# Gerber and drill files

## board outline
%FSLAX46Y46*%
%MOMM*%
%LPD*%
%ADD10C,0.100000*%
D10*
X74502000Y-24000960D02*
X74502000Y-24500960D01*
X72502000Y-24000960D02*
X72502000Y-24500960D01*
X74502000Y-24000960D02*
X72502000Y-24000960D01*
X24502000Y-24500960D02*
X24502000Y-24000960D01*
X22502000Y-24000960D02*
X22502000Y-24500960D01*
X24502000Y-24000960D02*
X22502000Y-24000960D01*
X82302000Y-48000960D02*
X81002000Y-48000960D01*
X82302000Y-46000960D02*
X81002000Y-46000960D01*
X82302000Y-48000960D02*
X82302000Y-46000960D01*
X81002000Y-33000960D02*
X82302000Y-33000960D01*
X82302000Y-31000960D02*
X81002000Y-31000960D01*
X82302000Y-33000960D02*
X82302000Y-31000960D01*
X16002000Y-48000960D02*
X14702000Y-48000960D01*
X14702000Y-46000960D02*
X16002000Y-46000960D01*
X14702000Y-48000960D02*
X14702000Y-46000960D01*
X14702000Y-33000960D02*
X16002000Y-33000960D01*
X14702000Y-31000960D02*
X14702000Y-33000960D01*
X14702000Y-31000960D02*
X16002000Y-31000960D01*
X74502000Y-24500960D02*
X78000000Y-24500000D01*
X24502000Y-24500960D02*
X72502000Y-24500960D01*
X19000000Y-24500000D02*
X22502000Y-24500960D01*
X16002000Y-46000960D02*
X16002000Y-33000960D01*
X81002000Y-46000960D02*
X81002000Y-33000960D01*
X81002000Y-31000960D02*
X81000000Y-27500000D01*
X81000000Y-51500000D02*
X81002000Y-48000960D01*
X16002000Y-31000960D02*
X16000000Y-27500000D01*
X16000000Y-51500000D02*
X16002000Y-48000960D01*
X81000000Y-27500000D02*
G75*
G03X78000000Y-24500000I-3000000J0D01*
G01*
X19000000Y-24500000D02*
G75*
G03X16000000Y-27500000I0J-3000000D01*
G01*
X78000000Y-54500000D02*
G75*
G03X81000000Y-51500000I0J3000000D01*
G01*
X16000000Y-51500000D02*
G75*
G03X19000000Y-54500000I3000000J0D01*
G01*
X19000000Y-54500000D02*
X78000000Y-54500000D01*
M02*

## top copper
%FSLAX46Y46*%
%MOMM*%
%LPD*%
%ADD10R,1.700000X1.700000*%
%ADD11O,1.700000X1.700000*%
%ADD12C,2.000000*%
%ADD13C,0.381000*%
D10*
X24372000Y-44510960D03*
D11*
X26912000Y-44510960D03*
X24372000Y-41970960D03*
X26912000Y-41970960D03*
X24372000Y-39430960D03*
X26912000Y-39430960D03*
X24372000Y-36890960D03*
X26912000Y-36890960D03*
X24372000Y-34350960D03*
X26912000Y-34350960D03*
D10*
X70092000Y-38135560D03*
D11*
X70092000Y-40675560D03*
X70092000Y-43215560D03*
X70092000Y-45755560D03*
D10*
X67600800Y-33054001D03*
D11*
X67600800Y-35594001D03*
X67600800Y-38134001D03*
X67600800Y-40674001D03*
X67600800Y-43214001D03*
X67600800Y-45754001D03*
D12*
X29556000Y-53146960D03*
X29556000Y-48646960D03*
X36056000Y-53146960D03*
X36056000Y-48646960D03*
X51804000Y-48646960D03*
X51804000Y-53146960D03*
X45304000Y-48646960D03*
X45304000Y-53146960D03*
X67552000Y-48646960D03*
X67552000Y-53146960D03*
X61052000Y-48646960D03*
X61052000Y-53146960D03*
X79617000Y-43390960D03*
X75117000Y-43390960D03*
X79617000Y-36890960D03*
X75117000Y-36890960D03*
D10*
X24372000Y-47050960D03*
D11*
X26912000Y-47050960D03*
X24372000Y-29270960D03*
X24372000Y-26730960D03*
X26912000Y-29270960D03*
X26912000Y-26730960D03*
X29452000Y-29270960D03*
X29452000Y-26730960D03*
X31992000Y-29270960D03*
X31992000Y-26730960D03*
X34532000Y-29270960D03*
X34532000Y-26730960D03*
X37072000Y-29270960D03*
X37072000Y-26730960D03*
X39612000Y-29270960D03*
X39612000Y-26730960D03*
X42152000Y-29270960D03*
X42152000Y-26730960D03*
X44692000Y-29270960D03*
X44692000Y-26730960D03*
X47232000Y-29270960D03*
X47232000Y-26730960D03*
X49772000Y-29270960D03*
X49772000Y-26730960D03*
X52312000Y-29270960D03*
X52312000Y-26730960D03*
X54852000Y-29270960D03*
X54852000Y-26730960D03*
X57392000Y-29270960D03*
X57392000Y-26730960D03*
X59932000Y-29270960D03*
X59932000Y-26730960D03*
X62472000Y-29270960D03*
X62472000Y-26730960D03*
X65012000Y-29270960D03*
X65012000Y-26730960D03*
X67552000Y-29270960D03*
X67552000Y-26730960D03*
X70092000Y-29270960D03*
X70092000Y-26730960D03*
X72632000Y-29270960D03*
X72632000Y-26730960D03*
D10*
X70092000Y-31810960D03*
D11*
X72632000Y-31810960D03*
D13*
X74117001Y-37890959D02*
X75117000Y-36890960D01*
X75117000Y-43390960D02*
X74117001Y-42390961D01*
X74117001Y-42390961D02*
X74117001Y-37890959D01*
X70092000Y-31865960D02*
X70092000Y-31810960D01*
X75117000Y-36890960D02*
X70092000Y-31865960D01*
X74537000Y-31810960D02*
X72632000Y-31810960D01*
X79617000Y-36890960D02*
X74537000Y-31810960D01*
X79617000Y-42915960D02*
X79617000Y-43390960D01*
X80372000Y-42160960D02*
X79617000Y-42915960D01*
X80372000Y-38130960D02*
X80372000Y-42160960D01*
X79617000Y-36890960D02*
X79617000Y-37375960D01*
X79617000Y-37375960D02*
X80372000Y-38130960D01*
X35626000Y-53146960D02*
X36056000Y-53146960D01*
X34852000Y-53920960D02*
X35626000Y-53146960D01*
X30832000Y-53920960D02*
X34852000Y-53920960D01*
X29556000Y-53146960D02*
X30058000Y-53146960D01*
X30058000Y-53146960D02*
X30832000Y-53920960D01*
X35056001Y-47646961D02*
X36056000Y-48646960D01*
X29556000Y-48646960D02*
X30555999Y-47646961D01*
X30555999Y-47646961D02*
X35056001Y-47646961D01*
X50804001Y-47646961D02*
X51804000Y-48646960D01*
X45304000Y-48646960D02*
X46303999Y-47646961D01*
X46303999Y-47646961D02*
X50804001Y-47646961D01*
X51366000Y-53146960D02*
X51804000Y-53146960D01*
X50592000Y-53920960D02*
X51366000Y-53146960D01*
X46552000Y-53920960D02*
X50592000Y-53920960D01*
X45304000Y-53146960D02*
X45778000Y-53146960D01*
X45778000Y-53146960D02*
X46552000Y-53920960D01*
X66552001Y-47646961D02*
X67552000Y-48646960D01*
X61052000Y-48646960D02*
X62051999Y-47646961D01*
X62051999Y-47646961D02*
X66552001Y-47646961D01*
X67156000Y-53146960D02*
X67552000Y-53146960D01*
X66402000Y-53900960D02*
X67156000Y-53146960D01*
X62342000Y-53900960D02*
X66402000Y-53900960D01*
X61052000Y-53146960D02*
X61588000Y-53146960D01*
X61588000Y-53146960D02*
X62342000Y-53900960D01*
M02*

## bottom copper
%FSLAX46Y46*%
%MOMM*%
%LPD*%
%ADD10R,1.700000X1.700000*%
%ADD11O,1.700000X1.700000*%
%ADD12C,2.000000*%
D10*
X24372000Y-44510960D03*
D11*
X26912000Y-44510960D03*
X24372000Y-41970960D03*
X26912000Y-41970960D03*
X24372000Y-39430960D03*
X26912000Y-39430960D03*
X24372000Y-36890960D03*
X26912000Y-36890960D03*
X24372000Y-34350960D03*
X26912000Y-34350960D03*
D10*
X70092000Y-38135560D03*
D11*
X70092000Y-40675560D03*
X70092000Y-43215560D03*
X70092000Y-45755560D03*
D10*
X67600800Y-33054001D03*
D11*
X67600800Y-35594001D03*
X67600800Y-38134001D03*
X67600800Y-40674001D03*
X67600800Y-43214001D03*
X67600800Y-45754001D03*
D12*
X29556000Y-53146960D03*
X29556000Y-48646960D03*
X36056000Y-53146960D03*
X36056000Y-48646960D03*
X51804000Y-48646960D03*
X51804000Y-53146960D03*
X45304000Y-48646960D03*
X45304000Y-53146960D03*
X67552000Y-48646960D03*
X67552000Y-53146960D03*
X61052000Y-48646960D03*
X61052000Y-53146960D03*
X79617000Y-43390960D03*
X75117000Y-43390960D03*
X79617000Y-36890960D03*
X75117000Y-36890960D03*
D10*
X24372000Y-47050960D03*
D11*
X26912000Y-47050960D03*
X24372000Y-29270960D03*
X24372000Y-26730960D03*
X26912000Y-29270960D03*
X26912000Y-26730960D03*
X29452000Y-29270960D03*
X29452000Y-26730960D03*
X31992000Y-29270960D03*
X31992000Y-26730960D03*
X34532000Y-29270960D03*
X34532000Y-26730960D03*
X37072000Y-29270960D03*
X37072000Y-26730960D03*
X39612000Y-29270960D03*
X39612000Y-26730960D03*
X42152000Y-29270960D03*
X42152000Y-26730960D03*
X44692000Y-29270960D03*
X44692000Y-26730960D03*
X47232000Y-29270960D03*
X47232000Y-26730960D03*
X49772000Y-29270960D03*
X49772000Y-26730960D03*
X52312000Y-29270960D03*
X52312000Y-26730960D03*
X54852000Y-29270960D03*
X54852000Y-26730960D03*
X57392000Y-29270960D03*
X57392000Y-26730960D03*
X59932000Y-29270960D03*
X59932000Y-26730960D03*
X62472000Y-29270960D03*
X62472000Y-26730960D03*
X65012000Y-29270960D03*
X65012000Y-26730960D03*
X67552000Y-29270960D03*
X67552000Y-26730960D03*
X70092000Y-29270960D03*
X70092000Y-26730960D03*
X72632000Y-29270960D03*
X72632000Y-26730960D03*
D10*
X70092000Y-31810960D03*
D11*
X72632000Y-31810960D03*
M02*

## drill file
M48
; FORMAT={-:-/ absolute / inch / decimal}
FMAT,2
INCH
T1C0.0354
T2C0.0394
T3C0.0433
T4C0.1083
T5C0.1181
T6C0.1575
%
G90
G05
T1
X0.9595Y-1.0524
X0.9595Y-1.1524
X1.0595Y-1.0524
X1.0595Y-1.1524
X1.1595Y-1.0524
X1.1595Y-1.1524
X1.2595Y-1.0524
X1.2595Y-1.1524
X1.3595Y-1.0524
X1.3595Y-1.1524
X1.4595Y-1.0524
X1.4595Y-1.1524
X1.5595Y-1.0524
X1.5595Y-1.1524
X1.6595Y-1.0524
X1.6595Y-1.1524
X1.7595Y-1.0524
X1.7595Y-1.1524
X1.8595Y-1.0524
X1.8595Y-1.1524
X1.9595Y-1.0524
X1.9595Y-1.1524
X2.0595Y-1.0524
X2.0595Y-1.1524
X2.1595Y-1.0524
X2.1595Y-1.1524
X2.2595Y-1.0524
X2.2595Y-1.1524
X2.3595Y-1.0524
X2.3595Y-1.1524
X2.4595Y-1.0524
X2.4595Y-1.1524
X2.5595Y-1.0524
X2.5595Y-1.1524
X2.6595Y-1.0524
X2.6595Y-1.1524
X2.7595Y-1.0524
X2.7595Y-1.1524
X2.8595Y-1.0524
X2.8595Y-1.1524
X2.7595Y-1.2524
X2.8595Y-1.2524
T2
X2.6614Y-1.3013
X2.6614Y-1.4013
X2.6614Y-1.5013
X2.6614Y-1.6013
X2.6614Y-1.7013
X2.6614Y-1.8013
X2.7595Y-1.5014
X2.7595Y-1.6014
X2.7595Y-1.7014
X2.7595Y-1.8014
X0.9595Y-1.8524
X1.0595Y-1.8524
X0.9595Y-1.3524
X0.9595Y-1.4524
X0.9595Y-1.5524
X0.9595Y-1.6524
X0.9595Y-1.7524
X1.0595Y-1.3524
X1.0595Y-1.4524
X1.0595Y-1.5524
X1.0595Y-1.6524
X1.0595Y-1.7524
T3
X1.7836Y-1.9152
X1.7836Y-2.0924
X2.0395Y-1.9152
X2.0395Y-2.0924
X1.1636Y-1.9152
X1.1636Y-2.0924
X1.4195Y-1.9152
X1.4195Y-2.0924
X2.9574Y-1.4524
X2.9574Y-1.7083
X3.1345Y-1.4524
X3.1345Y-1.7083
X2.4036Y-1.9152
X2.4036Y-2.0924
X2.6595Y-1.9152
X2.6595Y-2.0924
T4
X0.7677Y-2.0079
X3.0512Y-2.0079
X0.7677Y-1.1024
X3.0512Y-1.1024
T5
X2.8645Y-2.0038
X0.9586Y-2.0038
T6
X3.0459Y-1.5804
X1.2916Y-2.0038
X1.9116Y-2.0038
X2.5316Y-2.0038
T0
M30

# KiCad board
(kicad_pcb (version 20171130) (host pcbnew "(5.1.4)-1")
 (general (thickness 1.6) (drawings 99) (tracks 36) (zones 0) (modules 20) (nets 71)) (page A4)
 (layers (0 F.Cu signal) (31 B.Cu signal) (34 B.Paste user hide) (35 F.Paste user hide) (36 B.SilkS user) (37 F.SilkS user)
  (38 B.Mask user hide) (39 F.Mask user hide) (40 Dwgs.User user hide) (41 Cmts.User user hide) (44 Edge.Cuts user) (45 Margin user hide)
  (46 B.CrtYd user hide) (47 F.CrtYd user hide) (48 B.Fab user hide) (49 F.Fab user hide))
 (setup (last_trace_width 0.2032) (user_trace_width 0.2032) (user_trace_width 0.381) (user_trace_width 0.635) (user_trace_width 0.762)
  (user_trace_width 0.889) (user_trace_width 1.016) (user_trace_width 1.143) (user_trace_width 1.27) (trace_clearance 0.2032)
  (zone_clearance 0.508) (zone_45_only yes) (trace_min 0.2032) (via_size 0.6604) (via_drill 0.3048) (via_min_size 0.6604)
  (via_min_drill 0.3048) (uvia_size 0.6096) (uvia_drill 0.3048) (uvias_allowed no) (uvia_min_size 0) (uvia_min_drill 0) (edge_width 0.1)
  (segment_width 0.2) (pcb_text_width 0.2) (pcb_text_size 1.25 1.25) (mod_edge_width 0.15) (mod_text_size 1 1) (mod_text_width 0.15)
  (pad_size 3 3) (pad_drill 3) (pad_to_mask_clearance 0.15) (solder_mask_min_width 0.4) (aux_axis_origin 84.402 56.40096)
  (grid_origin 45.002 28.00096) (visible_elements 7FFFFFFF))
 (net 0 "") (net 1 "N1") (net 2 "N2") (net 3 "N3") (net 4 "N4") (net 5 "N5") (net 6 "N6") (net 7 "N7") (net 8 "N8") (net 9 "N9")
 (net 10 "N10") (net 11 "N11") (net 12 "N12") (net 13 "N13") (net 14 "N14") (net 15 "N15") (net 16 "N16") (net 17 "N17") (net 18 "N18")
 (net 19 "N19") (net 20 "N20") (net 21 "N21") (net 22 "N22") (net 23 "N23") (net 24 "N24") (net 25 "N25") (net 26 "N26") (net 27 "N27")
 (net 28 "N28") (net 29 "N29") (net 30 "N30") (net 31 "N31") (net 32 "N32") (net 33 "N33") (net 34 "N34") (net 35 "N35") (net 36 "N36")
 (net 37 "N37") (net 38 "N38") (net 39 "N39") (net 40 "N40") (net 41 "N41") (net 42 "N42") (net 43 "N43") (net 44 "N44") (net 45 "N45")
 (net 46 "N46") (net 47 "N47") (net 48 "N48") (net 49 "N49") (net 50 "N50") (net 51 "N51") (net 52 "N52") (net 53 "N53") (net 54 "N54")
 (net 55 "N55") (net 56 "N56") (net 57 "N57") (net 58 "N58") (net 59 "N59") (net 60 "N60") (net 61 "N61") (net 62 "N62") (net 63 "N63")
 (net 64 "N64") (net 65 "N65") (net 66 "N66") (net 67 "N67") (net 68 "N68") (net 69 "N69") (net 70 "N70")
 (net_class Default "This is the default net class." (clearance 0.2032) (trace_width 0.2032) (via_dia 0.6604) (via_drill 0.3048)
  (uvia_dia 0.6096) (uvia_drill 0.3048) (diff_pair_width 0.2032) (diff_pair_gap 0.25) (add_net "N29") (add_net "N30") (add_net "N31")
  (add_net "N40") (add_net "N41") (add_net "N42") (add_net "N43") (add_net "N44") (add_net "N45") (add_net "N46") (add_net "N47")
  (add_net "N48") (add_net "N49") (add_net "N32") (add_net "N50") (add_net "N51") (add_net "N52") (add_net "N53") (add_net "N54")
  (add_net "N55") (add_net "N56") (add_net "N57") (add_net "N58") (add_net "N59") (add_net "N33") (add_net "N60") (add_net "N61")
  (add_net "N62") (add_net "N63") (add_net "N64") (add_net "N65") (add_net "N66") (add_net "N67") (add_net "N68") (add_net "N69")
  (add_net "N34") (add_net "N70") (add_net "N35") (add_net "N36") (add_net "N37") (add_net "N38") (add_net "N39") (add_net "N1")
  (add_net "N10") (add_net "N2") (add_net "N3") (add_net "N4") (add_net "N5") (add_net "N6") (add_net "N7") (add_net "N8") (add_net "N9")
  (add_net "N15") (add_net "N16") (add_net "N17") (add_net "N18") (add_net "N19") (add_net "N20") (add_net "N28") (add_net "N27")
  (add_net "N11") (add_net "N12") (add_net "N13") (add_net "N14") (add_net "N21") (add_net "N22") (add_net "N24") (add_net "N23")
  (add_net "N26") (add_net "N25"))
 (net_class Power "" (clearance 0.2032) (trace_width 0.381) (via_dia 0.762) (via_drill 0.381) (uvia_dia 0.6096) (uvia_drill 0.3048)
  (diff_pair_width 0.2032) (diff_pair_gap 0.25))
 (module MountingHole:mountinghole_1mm (layer F.Cu) (at 77.33862 39.95166)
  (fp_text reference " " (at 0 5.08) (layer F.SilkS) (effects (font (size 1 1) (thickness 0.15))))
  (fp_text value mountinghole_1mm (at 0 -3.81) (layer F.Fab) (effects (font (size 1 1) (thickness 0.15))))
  (pad "" np_thru_hole circle (at 0.02838 0.1893) (size 4 4) (drill 4) (layers *.Cu *.Mask) (zone_connect 0)))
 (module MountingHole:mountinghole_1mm (layer F.Cu) (at 24.35676 50.90668)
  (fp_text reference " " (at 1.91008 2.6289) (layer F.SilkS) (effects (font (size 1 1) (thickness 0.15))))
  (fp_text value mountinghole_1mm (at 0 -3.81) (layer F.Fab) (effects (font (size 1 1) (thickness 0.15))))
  (pad "" np_thru_hole circle (at -0.00776 -0.00972) (size 3 3) (drill 3) (layers *.Cu *.Mask)))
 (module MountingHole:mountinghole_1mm (layer F.Cu) (at 72.74376 50.90668)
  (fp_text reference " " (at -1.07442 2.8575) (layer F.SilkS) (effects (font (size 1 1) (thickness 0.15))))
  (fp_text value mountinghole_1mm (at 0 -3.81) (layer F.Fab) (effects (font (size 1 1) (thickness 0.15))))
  (pad "" np_thru_hole circle (at 0.01524 -0.00972) (size 3 3) (drill 3) (layers *.Cu *.Mask)))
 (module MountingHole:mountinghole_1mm (layer F.Cu) (at 64.29826 50.90414)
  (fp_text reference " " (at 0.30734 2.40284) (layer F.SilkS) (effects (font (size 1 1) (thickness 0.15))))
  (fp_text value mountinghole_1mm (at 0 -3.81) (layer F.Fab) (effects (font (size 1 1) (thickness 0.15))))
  (pad "" np_thru_hole circle (at 0.00374 -0.00718) (size 4 4) (drill 4) (layers *.Cu *.Mask) (zone_connect 0)))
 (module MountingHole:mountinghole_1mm (layer F.Cu) (at 48.51978 50.90414)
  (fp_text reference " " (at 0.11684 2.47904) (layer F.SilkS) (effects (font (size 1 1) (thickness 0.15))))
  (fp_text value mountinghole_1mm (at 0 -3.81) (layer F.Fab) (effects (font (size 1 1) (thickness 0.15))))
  (pad "" np_thru_hole circle (at 0.03422 -0.00718) (size 4 4) (drill 4) (layers *.Cu *.Mask) (zone_connect 0)))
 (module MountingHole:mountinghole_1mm (layer F.Cu) (at 32.78956 50.89398)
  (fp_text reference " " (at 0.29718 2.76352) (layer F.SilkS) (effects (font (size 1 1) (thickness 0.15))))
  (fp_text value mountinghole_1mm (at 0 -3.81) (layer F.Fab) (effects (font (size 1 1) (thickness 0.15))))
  (pad "" np_thru_hole circle (at 0.01644 0.00298) (size 4 4) (drill 4) (layers *.Cu *.Mask) (zone_connect 0)))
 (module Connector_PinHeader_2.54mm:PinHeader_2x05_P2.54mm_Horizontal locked (layer B.Cu) (at 24.372 44.51096)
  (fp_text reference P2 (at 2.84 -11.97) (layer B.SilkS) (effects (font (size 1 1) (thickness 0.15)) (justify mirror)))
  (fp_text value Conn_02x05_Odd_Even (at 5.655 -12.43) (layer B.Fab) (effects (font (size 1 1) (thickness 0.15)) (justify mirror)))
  (pad 1 thru_hole rect (at 0 0) (size 1.7 1.7) (drill 1) (layers *.Cu *.Mask) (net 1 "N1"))
  (pad 2 thru_hole oval (at 2.54 0) (size 1.7 1.7) (drill 1) (layers *.Cu *.Mask) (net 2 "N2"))
  (pad 3 thru_hole oval (at 0 -2.54) (size 1.7 1.7) (drill 1) (layers *.Cu *.Mask) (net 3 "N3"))
  (pad 4 thru_hole oval (at 2.54 -2.54) (size 1.7 1.7) (drill 1) (layers *.Cu *.Mask) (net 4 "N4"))
  (pad 5 thru_hole oval (at 0 -5.08) (size 1.7 1.7) (drill 1) (layers *.Cu *.Mask) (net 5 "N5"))
  (pad 6 thru_hole oval (at 2.54 -5.08) (size 1.7 1.7) (drill 1) (layers *.Cu *.Mask) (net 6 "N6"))
  (pad 7 thru_hole oval (at 0 -7.62) (size 1.7 1.7) (drill 1) (layers *.Cu *.Mask) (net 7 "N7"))
  (pad 8 thru_hole oval (at 2.54 -7.62) (size 1.7 1.7) (drill 1) (layers *.Cu *.Mask) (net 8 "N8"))
  (pad 9 thru_hole oval (at 0 -10.16) (size 1.7 1.7) (drill 1) (layers *.Cu *.Mask) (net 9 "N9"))
  (pad 10 thru_hole oval (at 2.54 -10.16) (size 1.7 1.7) (drill 1) (layers *.Cu *.Mask) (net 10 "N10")))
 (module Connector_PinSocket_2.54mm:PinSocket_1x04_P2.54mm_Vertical (layer B.Cu) (at 70.092 38.13556 180)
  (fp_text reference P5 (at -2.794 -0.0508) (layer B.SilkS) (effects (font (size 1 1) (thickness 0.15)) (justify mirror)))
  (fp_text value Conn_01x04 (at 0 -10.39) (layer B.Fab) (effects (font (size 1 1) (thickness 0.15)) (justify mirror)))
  (pad 1 thru_hole rect (at 0 0 180) (size 1.7 1.7) (drill 1) (layers *.Cu *.Mask) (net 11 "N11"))
  (pad 2 thru_hole oval (at 0 -2.54 180) (size 1.7 1.7) (drill 1) (layers *.Cu *.Mask) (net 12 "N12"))
  (pad 3 thru_hole oval (at 0 -5.08 180) (size 1.7 1.7) (drill 1) (layers *.Cu *.Mask) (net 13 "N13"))
  (pad 4 thru_hole oval (at 0 -7.62 180) (size 1.7 1.7) (drill 1) (layers *.Cu *.Mask) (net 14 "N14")))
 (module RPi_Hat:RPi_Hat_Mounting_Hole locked (layer F.Cu) (at 19.5 51)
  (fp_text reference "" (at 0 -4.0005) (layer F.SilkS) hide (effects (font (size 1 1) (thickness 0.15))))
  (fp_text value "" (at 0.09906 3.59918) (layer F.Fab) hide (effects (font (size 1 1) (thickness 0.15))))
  (pad "" np_thru_hole circle (at 0 0) (size 2.75 2.75) (drill 2.75) (layers *.Cu *.Mask) (solder_mask_margin 1.725) (clearance 1.725)))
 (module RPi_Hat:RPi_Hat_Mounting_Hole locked (layer F.Cu) (at 77.5 28)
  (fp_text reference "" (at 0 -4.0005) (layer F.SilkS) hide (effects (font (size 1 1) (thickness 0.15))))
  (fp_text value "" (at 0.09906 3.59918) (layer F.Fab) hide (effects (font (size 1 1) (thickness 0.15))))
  (pad "" np_thru_hole circle (at 0 0) (size 2.75 2.75) (drill 2.75) (layers *.Cu *.Mask) (solder_mask_margin 1.725) (clearance 1.725)))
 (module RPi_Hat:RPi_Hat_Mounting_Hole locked (layer F.Cu) (at 77.5 51)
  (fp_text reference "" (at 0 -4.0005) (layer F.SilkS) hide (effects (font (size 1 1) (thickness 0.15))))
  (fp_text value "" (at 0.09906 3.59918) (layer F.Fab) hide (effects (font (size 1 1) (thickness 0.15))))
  (pad "" np_thru_hole circle (at 0 0) (size 2.75 2.75) (drill 2.75) (layers *.Cu *.Mask) (solder_mask_margin 1.725) (clearance 1.725)))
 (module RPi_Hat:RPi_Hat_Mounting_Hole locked (layer F.Cu) (at 19.5 28)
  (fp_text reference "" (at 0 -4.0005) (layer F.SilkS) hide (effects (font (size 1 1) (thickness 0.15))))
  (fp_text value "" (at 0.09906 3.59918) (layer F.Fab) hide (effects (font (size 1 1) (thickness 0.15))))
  (pad "" np_thru_hole circle (at 0 0) (size 2.75 2.75) (drill 2.75) (layers *.Cu *.Mask) (solder_mask_margin 1.725) (clearance 1.725)))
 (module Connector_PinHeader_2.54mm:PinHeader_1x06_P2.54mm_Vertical (layer F.Cu) (at 67.6008 33.054001)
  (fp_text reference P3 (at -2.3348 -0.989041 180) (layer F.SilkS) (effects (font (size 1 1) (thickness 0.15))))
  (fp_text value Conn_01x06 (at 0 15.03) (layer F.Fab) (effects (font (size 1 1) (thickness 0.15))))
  (pad 1 thru_hole rect (at 0 0) (size 1.7 1.7) (drill 1) (layers *.Cu *.Mask) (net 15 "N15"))
  (pad 2 thru_hole oval (at 0 2.54) (size 1.7 1.7) (drill 1) (layers *.Cu *.Mask) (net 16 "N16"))
  (pad 3 thru_hole oval (at 0 5.08) (size 1.7 1.7) (drill 1) (layers *.Cu *.Mask) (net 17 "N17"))
  (pad 4 thru_hole oval (at 0 7.62) (size 1.7 1.7) (drill 1) (layers *.Cu *.Mask) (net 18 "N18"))
  (pad 5 thru_hole oval (at 0 10.16) (size 1.7 1.7) (drill 1) (layers *.Cu *.Mask) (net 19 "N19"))
  (pad 6 thru_hole oval (at 0 12.7) (size 1.7 1.7) (drill 1) (layers *.Cu *.Mask) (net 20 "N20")))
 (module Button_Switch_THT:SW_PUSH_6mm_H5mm (layer F.Cu) (at 36.056 53.14696 180)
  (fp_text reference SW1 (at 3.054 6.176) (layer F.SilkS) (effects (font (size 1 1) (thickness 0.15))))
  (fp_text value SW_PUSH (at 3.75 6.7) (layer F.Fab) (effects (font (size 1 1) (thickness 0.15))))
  (pad 1 thru_hole circle (at 6.5 0 270) (size 2 2) (drill 1.1) (layers *.Cu *.Mask) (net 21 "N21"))
  (pad 2 thru_hole circle (at 6.5 4.5 270) (size 2 2) (drill 1.1) (layers *.Cu *.Mask) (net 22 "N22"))
  (pad 1 thru_hole circle (at 0 0 270) (size 2 2) (drill 1.1) (layers *.Cu *.Mask) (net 21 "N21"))
  (pad 2 thru_hole circle (at 0 4.5 270) (size 2 2) (drill 1.1) (layers *.Cu *.Mask) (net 22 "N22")))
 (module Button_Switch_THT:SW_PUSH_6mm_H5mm (layer F.Cu) (at 51.804 53.14696 180)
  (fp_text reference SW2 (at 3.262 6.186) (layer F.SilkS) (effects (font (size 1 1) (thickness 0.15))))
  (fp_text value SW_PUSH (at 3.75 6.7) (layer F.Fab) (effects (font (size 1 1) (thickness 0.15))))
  (pad 2 thru_hole circle (at 0 4.5 270) (size 2 2) (drill 1.1) (layers *.Cu *.Mask) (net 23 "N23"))
  (pad 1 thru_hole circle (at 0 0 270) (size 2 2) (drill 1.1) (layers *.Cu *.Mask) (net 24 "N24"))
  (pad 2 thru_hole circle (at 6.5 4.5 270) (size 2 2) (drill 1.1) (layers *.Cu *.Mask) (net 23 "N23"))
  (pad 1 thru_hole circle (at 6.5 0 270) (size 2 2) (drill 1.1) (layers *.Cu *.Mask) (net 24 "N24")))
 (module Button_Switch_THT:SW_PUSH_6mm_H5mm (layer F.Cu) (at 67.552 53.14696 180)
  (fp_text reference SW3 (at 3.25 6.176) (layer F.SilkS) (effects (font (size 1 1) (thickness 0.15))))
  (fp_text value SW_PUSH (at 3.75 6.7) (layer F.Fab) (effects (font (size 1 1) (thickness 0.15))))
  (pad 2 thru_hole circle (at 0 4.5 270) (size 2 2) (drill 1.1) (layers *.Cu *.Mask) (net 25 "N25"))
  (pad 1 thru_hole circle (at 0 0 270) (size 2 2) (drill 1.1) (layers *.Cu *.Mask) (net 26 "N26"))
  (pad 2 thru_hole circle (at 6.5 4.5 270) (size 2 2) (drill 1.1) (layers *.Cu *.Mask) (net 25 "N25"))
  (pad 1 thru_hole circle (at 6.5 0 270) (size 2 2) (drill 1.1) (layers *.Cu *.Mask) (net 26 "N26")))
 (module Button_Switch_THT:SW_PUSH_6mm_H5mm (layer F.Cu) (at 79.617 36.89096 270)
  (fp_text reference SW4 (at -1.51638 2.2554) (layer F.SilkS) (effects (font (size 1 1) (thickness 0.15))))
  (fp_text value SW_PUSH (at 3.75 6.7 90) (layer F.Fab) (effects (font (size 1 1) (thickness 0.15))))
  (pad 1 thru_hole circle (at 6.5 0) (size 2 2) (drill 1.1) (layers *.Cu *.Mask) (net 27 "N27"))
  (pad 2 thru_hole circle (at 6.5 4.5) (size 2 2) (drill 1.1) (layers *.Cu *.Mask) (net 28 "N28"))
  (pad 1 thru_hole circle (at 0 0) (size 2 2) (drill 1.1) (layers *.Cu *.Mask) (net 27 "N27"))
  (pad 2 thru_hole circle (at 0 4.5) (size 2 2) (drill 1.1) (layers *.Cu *.Mask) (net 28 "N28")))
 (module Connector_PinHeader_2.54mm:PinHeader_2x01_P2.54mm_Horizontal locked (layer B.Cu) (at 24.372 47.05096)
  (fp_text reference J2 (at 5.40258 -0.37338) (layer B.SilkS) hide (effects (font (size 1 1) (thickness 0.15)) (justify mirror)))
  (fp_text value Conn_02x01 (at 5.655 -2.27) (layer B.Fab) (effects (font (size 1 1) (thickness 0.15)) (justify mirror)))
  (pad 1 thru_hole rect (at 0 0) (size 1.7 1.7) (drill 1) (layers *.Cu *.Mask) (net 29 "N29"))
  (pad 2 thru_hole oval (at 2.54 0) (size 1.7 1.7) (drill 1) (layers *.Cu *.Mask) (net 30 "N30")))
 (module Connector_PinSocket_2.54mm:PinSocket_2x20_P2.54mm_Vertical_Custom (layer B.Cu) (at 24.372 29.27096 270)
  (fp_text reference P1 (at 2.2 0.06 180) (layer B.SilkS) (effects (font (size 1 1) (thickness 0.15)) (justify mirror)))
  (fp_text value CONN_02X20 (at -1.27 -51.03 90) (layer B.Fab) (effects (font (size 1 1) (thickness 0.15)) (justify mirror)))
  (pad 1 thru_hole oval (at 0 0 270) (size 1.7 1.7) (drill 0.9) (layers *.Cu *.Mask) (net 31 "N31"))
  (pad 2 thru_hole oval (at -2.54 0 270) (size 1.7 1.7) (drill 0.9) (layers *.Cu *.Mask) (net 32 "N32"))
  (pad 3 thru_hole oval (at 0 -2.54 270) (size 1.7 1.7) (drill 0.9) (layers *.Cu *.Mask) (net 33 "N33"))
  (pad 4 thru_hole oval (at -2.54 -2.54 270) (size 1.7 1.7) (drill 0.9) (layers *.Cu *.Mask) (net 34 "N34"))
  (pad 5 thru_hole oval (at 0 -5.08 270) (size 1.7 1.7) (drill 0.9) (layers *.Cu *.Mask) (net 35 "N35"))
  (pad 6 thru_hole oval (at -2.54 -5.08 270) (size 1.7 1.7) (drill 0.9) (layers *.Cu *.Mask) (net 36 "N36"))
  (pad 7 thru_hole oval (at 0 -7.62 270) (size 1.7 1.7) (drill 0.9) (layers *.Cu *.Mask) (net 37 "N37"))
  (pad 8 thru_hole oval (at -2.54 -7.62 270) (size 1.7 1.7) (drill 0.9) (layers *.Cu *.Mask) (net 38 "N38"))
  (pad 9 thru_hole oval (at 0 -10.16 270) (size 1.7 1.7) (drill 0.9) (layers *.Cu *.Mask) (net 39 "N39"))
  (pad 10 thru_hole oval (at -2.54 -10.16 270) (size 1.7 1.7) (drill 0.9) (layers *.Cu *.Mask) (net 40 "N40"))
  (pad 11 thru_hole oval (at 0 -12.7 270) (size 1.7 1.7) (drill 0.9) (layers *.Cu *.Mask) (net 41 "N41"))
  (pad 12 thru_hole oval (at -2.54 -12.7 270) (size 1.7 1.7) (drill 0.9) (layers *.Cu *.Mask) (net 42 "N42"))
  (pad 13 thru_hole oval (at 0 -15.24 270) (size 1.7 1.7) (drill 0.9) (layers *.Cu *.Mask) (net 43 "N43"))
  (pad 14 thru_hole oval (at -2.54 -15.24 270) (size 1.7 1.7) (drill 0.9) (layers *.Cu *.Mask) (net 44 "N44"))
  (pad 15 thru_hole oval (at 0 -17.78 270) (size 1.7 1.7) (drill 0.9) (layers *.Cu *.Mask) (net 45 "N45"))
  (pad 16 thru_hole oval (at -2.54 -17.78 270) (size 1.7 1.7) (drill 0.9) (layers *.Cu *.Mask) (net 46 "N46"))
  (pad 17 thru_hole oval (at 0 -20.32 270) (size 1.7 1.7) (drill 0.9) (layers *.Cu *.Mask) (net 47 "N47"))
  (pad 18 thru_hole oval (at -2.54 -20.32 270) (size 1.7 1.7) (drill 0.9) (layers *.Cu *.Mask) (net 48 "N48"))
  (pad 19 thru_hole oval (at 0 -22.86 270) (size 1.7 1.7) (drill 0.9) (layers *.Cu *.Mask) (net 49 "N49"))
  (pad 20 thru_hole oval (at -2.54 -22.86 270) (size 1.7 1.7) (drill 0.9) (layers *.Cu *.Mask) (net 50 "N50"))
  (pad 21 thru_hole oval (at 0 -25.4 270) (size 1.7 1.7) (drill 0.9) (layers *.Cu *.Mask) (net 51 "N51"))
  (pad 22 thru_hole oval (at -2.54 -25.4 270) (size 1.7 1.7) (drill 0.9) (layers *.Cu *.Mask) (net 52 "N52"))
  (pad 23 thru_hole oval (at 0 -27.94 270) (size 1.7 1.7) (drill 0.9) (layers *.Cu *.Mask) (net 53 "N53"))
  (pad 24 thru_hole oval (at -2.54 -27.94 270) (size 1.7 1.7) (drill 0.9) (layers *.Cu *.Mask) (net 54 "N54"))
  (pad 25 thru_hole oval (at 0 -30.48 270) (size 1.7 1.7) (drill 0.9) (layers *.Cu *.Mask) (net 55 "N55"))
  (pad 26 thru_hole oval (at -2.54 -30.48 270) (size 1.7 1.7) (drill 0.9) (layers *.Cu *.Mask) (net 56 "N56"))
  (pad 27 thru_hole oval (at 0 -33.02 270) (size 1.7 1.7) (drill 0.9) (layers *.Cu *.Mask) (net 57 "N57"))
  (pad 28 thru_hole oval (at -2.54 -33.02 270) (size 1.7 1.7) (drill 0.9) (layers *.Cu *.Mask) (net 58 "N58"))
  (pad 29 thru_hole oval (at 0 -35.56 270) (size 1.7 1.7) (drill 0.9) (layers *.Cu *.Mask) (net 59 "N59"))
  (pad 30 thru_hole oval (at -2.54 -35.56 270) (size 1.7 1.7) (drill 0.9) (layers *.Cu *.Mask) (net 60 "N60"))
  (pad 31 thru_hole oval (at 0 -38.1 270) (size 1.7 1.7) (drill 0.9) (layers *.Cu *.Mask) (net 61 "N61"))
  (pad 32 thru_hole oval (at -2.54 -38.1 270) (size 1.7 1.7) (drill 0.9) (layers *.Cu *.Mask) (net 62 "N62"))
  (pad 33 thru_hole oval (at 0 -40.64 270) (size 1.7 1.7) (drill 0.9) (layers *.Cu *.Mask) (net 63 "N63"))
  (pad 34 thru_hole oval (at -2.54 -40.64 270) (size 1.7 1.7) (drill 0.9) (layers *.Cu *.Mask) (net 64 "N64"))
  (pad 35 thru_hole oval (at 0 -43.18 270) (size 1.7 1.7) (drill 0.9) (layers *.Cu *.Mask) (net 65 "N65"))
  (pad 36 thru_hole oval (at -2.54 -43.18 270) (size 1.7 1.7) (drill 0.9) (layers *.Cu *.Mask) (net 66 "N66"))
  (pad 37 thru_hole oval (at 0 -45.72 270) (size 1.7 1.7) (drill 0.9) (layers *.Cu *.Mask) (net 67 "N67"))
  (pad 38 thru_hole oval (at -2.54 -45.72 270) (size 1.7 1.7) (drill 0.9) (layers *.Cu *.Mask) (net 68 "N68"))
  (pad 39 thru_hole oval (at 0 -48.26 270) (size 1.7 1.7) (drill 0.9) (layers *.Cu *.Mask) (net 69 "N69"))
  (pad 40 thru_hole oval (at -2.54 -48.26 270) (size 1.7 1.7) (drill 0.9) (layers *.Cu *.Mask) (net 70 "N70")))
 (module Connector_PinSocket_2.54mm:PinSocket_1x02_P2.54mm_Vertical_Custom (layer B.Cu) (at 70.092 31.81096 270)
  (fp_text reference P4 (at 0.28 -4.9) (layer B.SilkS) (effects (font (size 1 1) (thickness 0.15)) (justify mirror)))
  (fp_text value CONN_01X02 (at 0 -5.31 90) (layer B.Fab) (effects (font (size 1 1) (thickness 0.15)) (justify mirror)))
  (pad 1 thru_hole rect (at 0 0 270) (size 1.7 1.7) (drill 0.9) (layers *.Cu *.Mask) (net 28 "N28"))
  (pad 2 thru_hole oval (at 0 -2.54 270) (size 1.7 1.7) (drill 0.9) (layers *.Cu *.Mask) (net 27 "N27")))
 (gr_line (start 74.502 24.00096) (end 74.502 24.50096) (layer Edge.Cuts) (width 0.1))
 (gr_line (start 72.502 24.00096) (end 72.502 24.50096) (layer Edge.Cuts) (width 0.1))
 (gr_line (start 74.502 24.00096) (end 72.502 24.00096) (layer Edge.Cuts) (width 0.1))
 (gr_line (start 24.502 24.50096) (end 24.502 24.00096) (layer Edge.Cuts) (width 0.1))
 (gr_line (start 22.502 24.00096) (end 22.502 24.50096) (layer Edge.Cuts) (width 0.1))
 (gr_line (start 24.502 24.00096) (end 22.502 24.00096) (layer Edge.Cuts) (width 0.1))
 (gr_line (start 82.302 48.00096) (end 81.002 48.00096) (layer Edge.Cuts) (width 0.1))
 (gr_line (start 82.302 46.00096) (end 81.002 46.00096) (layer Edge.Cuts) (width 0.1))
 (gr_line (start 82.302 48.00096) (end 82.302 46.00096) (layer Edge.Cuts) (width 0.1))
 (gr_line (start 81.002 33.00096) (end 82.302 33.00096) (layer Edge.Cuts) (width 0.1))
 (gr_line (start 82.302 31.00096) (end 81.002 31.00096) (layer Edge.Cuts) (width 0.1))
 (gr_line (start 82.302 33.00096) (end 82.302 31.00096) (layer Edge.Cuts) (width 0.1))
 (gr_line (start 16.002 48.00096) (end 14.702 48.00096) (layer Edge.Cuts) (width 0.1))
 (gr_line (start 14.702 46.00096) (end 16.002 46.00096) (layer Edge.Cuts) (width 0.1))
 (gr_line (start 14.702 48.00096) (end 14.702 46.00096) (layer Edge.Cuts) (width 0.1))
 (gr_line (start 14.702 33.00096) (end 16.002 33.00096) (layer Edge.Cuts) (width 0.1))
 (gr_line (start 14.702 31.00096) (end 14.702 33.00096) (layer Edge.Cuts) (width 0.1))
 (gr_line (start 14.702 31.00096) (end 16.002 31.00096) (layer Edge.Cuts) (width 0.1))
 (gr_line (start 74.502 24.50096) (end 78 24.5) (layer Edge.Cuts) (width 0.1))
 (gr_line (start 24.502 24.50096) (end 72.502 24.50096) (layer Edge.Cuts) (width 0.1))
 (gr_line (start 19 24.5) (end 22.502 24.50096) (layer Edge.Cuts) (width 0.1))
 (gr_line (start 16.002 46.00096) (end 16.002 33.00096) (layer Edge.Cuts) (width 0.1))
 (gr_line (start 81.002 46.00096) (end 81.002 33.00096) (layer Edge.Cuts) (width 0.1))
 (gr_line (start 81.002 31.00096) (end 81 27.5) (layer Edge.Cuts) (width 0.1))
 (gr_line (start 81 51.5) (end 81.002 48.00096) (layer Edge.Cuts) (width 0.1))
 (gr_line (start 16.002 31.00096) (end 16 27.5) (layer Edge.Cuts) (width 0.1))
 (gr_line (start 16 51.5) (end 16.002 48.00096) (layer Edge.Cuts) (width 0.1))
 (gr_arc (start 78 27.5) (end 78 24.5) (angle 90) (layer Edge.Cuts) (width 0.1))
 (gr_arc (start 19 27.5) (end 16 27.5) (angle 90) (layer Edge.Cuts) (width 0.1))
 (gr_arc (start 78 51.5) (end 81 51.5) (angle 90) (layer Edge.Cuts) (width 0.1))
 (gr_arc (start 19 51.5) (end 19 54.5) (angle 90) (layer Edge.Cuts) (width 0.1))
 (gr_line (start 19 54.5) (end 78 54.5) (angle 90) (layer Edge.Cuts) (width 0.1))
 (segment (start 74.117001 37.890959) (end 75.117 36.89096) (width 0.381) (layer F.Cu) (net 28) (status 20))
 (segment (start 75.117 43.39096) (end 74.117001 42.390961) (width 0.381) (layer F.Cu) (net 28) (status 10))
 (segment (start 74.117001 42.390961) (end 74.117001 37.890959) (width 0.381) (layer F.Cu) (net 28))
 (segment (start 70.092 31.86596) (end 70.092 31.81096) (width 0.381) (layer F.Cu) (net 28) (status 30))
 (segment (start 75.117 36.89096) (end 70.092 31.86596) (width 0.381) (layer F.Cu) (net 28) (status 30))
 (segment (start 74.537 31.81096) (end 72.632 31.81096) (width 0.381) (layer F.Cu) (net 27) (status 20))
 (segment (start 79.617 36.89096) (end 74.537 31.81096) (width 0.381) (layer F.Cu) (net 27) (status 10))
 (segment (start 79.617 42.91596) (end 79.617 43.39096) (width 0.381) (layer F.Cu) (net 27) (status 30))
 (segment (start 80.372 42.16096) (end 79.617 42.91596) (width 0.381) (layer F.Cu) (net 27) (status 20))
 (segment (start 80.372 38.13096) (end 80.372 42.16096) (width 0.381) (layer F.Cu) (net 27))
 (segment (start 79.617 36.89096) (end 79.617 37.37596) (width 0.381) (layer F.Cu) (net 27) (status 30))
 (segment (start 79.617 37.37596) (end 80.372 38.13096) (width 0.381) (layer F.Cu) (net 27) (status 10))
 (segment (start 35.626 53.14696) (end 36.056 53.14696) (width 0.381) (layer F.Cu) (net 21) (status 30))
 (segment (start 34.852 53.92096) (end 35.626 53.14696) (width 0.381) (layer F.Cu) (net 21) (status 20))
 (segment (start 30.832 53.92096) (end 34.852 53.92096) (width 0.381) (layer F.Cu) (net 21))
 (segment (start 29.556 53.14696) (end 30.058 53.14696) (width 0.381) (layer F.Cu) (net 21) (status 30))
 (segment (start 30.058 53.14696) (end 30.832 53.92096) (width 0.381) (layer F.Cu) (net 21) (status 10))
 (segment (start 35.056001 47.646961) (end 36.056 48.64696) (width 0.381) (layer F.Cu) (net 22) (status 20))
 (segment (start 29.556 48.64696) (end 30.555999 47.646961) (width 0.381) (layer F.Cu) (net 22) (status 10))
 (segment (start 30.555999 47.646961) (end 35.056001 47.646961) (width 0.381) (layer F.Cu) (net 22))
 (segment (start 50.804001 47.646961) (end 51.804 48.64696) (width 0.381) (layer F.Cu) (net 23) (status 20))
 (segment (start 45.304 48.64696) (end 46.303999 47.646961) (width 0.381) (layer F.Cu) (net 23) (status 10))
 (segment (start 46.303999 47.646961) (end 50.804001 47.646961) (width 0.381) (layer F.Cu) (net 23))
 (segment (start 51.366 53.14696) (end 51.804 53.14696) (width 0.381) (layer F.Cu) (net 24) (status 30))
 (segment (start 50.592 53.92096) (end 51.366 53.14696) (width 0.381) (layer F.Cu) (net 24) (status 20))
 (segment (start 46.552 53.92096) (end 50.592 53.92096) (width 0.381) (layer F.Cu) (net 24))
 (segment (start 45.304 53.14696) (end 45.778 53.14696) (width 0.381) (layer F.Cu) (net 24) (status 30))
 (segment (start 45.778 53.14696) (end 46.552 53.92096) (width 0.381) (layer F.Cu) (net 24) (status 10))
 (segment (start 66.552001 47.646961) (end 67.552 48.64696) (width 0.381) (layer F.Cu) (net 25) (status 20))
 (segment (start 61.052 48.64696) (end 62.051999 47.646961) (width 0.381) (layer F.Cu) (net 25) (status 10))
 (segment (start 62.051999 47.646961) (end 66.552001 47.646961) (width 0.381) (layer F.Cu) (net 25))
 (segment (start 67.156 53.14696) (end 67.552 53.14696) (width 0.381) (layer F.Cu) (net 26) (status 30))
 (segment (start 66.402 53.90096) (end 67.156 53.14696) (width 0.381) (layer F.Cu) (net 26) (status 20))
 (segment (start 62.342 53.90096) (end 66.402 53.90096) (width 0.381) (layer F.Cu) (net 26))
 (segment (start 61.052 53.14696) (end 61.588 53.14696) (width 0.381) (layer F.Cu) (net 26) (status 30))
 (segment (start 61.588 53.14696) (end 62.342 53.90096) (width 0.381) (layer F.Cu) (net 26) (status 10))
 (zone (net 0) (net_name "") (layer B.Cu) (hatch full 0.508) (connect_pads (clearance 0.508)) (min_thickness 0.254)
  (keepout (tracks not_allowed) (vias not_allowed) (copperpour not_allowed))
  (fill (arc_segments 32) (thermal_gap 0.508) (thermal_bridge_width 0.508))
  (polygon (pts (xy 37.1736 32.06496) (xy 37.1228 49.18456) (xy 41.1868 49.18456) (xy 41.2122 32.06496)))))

